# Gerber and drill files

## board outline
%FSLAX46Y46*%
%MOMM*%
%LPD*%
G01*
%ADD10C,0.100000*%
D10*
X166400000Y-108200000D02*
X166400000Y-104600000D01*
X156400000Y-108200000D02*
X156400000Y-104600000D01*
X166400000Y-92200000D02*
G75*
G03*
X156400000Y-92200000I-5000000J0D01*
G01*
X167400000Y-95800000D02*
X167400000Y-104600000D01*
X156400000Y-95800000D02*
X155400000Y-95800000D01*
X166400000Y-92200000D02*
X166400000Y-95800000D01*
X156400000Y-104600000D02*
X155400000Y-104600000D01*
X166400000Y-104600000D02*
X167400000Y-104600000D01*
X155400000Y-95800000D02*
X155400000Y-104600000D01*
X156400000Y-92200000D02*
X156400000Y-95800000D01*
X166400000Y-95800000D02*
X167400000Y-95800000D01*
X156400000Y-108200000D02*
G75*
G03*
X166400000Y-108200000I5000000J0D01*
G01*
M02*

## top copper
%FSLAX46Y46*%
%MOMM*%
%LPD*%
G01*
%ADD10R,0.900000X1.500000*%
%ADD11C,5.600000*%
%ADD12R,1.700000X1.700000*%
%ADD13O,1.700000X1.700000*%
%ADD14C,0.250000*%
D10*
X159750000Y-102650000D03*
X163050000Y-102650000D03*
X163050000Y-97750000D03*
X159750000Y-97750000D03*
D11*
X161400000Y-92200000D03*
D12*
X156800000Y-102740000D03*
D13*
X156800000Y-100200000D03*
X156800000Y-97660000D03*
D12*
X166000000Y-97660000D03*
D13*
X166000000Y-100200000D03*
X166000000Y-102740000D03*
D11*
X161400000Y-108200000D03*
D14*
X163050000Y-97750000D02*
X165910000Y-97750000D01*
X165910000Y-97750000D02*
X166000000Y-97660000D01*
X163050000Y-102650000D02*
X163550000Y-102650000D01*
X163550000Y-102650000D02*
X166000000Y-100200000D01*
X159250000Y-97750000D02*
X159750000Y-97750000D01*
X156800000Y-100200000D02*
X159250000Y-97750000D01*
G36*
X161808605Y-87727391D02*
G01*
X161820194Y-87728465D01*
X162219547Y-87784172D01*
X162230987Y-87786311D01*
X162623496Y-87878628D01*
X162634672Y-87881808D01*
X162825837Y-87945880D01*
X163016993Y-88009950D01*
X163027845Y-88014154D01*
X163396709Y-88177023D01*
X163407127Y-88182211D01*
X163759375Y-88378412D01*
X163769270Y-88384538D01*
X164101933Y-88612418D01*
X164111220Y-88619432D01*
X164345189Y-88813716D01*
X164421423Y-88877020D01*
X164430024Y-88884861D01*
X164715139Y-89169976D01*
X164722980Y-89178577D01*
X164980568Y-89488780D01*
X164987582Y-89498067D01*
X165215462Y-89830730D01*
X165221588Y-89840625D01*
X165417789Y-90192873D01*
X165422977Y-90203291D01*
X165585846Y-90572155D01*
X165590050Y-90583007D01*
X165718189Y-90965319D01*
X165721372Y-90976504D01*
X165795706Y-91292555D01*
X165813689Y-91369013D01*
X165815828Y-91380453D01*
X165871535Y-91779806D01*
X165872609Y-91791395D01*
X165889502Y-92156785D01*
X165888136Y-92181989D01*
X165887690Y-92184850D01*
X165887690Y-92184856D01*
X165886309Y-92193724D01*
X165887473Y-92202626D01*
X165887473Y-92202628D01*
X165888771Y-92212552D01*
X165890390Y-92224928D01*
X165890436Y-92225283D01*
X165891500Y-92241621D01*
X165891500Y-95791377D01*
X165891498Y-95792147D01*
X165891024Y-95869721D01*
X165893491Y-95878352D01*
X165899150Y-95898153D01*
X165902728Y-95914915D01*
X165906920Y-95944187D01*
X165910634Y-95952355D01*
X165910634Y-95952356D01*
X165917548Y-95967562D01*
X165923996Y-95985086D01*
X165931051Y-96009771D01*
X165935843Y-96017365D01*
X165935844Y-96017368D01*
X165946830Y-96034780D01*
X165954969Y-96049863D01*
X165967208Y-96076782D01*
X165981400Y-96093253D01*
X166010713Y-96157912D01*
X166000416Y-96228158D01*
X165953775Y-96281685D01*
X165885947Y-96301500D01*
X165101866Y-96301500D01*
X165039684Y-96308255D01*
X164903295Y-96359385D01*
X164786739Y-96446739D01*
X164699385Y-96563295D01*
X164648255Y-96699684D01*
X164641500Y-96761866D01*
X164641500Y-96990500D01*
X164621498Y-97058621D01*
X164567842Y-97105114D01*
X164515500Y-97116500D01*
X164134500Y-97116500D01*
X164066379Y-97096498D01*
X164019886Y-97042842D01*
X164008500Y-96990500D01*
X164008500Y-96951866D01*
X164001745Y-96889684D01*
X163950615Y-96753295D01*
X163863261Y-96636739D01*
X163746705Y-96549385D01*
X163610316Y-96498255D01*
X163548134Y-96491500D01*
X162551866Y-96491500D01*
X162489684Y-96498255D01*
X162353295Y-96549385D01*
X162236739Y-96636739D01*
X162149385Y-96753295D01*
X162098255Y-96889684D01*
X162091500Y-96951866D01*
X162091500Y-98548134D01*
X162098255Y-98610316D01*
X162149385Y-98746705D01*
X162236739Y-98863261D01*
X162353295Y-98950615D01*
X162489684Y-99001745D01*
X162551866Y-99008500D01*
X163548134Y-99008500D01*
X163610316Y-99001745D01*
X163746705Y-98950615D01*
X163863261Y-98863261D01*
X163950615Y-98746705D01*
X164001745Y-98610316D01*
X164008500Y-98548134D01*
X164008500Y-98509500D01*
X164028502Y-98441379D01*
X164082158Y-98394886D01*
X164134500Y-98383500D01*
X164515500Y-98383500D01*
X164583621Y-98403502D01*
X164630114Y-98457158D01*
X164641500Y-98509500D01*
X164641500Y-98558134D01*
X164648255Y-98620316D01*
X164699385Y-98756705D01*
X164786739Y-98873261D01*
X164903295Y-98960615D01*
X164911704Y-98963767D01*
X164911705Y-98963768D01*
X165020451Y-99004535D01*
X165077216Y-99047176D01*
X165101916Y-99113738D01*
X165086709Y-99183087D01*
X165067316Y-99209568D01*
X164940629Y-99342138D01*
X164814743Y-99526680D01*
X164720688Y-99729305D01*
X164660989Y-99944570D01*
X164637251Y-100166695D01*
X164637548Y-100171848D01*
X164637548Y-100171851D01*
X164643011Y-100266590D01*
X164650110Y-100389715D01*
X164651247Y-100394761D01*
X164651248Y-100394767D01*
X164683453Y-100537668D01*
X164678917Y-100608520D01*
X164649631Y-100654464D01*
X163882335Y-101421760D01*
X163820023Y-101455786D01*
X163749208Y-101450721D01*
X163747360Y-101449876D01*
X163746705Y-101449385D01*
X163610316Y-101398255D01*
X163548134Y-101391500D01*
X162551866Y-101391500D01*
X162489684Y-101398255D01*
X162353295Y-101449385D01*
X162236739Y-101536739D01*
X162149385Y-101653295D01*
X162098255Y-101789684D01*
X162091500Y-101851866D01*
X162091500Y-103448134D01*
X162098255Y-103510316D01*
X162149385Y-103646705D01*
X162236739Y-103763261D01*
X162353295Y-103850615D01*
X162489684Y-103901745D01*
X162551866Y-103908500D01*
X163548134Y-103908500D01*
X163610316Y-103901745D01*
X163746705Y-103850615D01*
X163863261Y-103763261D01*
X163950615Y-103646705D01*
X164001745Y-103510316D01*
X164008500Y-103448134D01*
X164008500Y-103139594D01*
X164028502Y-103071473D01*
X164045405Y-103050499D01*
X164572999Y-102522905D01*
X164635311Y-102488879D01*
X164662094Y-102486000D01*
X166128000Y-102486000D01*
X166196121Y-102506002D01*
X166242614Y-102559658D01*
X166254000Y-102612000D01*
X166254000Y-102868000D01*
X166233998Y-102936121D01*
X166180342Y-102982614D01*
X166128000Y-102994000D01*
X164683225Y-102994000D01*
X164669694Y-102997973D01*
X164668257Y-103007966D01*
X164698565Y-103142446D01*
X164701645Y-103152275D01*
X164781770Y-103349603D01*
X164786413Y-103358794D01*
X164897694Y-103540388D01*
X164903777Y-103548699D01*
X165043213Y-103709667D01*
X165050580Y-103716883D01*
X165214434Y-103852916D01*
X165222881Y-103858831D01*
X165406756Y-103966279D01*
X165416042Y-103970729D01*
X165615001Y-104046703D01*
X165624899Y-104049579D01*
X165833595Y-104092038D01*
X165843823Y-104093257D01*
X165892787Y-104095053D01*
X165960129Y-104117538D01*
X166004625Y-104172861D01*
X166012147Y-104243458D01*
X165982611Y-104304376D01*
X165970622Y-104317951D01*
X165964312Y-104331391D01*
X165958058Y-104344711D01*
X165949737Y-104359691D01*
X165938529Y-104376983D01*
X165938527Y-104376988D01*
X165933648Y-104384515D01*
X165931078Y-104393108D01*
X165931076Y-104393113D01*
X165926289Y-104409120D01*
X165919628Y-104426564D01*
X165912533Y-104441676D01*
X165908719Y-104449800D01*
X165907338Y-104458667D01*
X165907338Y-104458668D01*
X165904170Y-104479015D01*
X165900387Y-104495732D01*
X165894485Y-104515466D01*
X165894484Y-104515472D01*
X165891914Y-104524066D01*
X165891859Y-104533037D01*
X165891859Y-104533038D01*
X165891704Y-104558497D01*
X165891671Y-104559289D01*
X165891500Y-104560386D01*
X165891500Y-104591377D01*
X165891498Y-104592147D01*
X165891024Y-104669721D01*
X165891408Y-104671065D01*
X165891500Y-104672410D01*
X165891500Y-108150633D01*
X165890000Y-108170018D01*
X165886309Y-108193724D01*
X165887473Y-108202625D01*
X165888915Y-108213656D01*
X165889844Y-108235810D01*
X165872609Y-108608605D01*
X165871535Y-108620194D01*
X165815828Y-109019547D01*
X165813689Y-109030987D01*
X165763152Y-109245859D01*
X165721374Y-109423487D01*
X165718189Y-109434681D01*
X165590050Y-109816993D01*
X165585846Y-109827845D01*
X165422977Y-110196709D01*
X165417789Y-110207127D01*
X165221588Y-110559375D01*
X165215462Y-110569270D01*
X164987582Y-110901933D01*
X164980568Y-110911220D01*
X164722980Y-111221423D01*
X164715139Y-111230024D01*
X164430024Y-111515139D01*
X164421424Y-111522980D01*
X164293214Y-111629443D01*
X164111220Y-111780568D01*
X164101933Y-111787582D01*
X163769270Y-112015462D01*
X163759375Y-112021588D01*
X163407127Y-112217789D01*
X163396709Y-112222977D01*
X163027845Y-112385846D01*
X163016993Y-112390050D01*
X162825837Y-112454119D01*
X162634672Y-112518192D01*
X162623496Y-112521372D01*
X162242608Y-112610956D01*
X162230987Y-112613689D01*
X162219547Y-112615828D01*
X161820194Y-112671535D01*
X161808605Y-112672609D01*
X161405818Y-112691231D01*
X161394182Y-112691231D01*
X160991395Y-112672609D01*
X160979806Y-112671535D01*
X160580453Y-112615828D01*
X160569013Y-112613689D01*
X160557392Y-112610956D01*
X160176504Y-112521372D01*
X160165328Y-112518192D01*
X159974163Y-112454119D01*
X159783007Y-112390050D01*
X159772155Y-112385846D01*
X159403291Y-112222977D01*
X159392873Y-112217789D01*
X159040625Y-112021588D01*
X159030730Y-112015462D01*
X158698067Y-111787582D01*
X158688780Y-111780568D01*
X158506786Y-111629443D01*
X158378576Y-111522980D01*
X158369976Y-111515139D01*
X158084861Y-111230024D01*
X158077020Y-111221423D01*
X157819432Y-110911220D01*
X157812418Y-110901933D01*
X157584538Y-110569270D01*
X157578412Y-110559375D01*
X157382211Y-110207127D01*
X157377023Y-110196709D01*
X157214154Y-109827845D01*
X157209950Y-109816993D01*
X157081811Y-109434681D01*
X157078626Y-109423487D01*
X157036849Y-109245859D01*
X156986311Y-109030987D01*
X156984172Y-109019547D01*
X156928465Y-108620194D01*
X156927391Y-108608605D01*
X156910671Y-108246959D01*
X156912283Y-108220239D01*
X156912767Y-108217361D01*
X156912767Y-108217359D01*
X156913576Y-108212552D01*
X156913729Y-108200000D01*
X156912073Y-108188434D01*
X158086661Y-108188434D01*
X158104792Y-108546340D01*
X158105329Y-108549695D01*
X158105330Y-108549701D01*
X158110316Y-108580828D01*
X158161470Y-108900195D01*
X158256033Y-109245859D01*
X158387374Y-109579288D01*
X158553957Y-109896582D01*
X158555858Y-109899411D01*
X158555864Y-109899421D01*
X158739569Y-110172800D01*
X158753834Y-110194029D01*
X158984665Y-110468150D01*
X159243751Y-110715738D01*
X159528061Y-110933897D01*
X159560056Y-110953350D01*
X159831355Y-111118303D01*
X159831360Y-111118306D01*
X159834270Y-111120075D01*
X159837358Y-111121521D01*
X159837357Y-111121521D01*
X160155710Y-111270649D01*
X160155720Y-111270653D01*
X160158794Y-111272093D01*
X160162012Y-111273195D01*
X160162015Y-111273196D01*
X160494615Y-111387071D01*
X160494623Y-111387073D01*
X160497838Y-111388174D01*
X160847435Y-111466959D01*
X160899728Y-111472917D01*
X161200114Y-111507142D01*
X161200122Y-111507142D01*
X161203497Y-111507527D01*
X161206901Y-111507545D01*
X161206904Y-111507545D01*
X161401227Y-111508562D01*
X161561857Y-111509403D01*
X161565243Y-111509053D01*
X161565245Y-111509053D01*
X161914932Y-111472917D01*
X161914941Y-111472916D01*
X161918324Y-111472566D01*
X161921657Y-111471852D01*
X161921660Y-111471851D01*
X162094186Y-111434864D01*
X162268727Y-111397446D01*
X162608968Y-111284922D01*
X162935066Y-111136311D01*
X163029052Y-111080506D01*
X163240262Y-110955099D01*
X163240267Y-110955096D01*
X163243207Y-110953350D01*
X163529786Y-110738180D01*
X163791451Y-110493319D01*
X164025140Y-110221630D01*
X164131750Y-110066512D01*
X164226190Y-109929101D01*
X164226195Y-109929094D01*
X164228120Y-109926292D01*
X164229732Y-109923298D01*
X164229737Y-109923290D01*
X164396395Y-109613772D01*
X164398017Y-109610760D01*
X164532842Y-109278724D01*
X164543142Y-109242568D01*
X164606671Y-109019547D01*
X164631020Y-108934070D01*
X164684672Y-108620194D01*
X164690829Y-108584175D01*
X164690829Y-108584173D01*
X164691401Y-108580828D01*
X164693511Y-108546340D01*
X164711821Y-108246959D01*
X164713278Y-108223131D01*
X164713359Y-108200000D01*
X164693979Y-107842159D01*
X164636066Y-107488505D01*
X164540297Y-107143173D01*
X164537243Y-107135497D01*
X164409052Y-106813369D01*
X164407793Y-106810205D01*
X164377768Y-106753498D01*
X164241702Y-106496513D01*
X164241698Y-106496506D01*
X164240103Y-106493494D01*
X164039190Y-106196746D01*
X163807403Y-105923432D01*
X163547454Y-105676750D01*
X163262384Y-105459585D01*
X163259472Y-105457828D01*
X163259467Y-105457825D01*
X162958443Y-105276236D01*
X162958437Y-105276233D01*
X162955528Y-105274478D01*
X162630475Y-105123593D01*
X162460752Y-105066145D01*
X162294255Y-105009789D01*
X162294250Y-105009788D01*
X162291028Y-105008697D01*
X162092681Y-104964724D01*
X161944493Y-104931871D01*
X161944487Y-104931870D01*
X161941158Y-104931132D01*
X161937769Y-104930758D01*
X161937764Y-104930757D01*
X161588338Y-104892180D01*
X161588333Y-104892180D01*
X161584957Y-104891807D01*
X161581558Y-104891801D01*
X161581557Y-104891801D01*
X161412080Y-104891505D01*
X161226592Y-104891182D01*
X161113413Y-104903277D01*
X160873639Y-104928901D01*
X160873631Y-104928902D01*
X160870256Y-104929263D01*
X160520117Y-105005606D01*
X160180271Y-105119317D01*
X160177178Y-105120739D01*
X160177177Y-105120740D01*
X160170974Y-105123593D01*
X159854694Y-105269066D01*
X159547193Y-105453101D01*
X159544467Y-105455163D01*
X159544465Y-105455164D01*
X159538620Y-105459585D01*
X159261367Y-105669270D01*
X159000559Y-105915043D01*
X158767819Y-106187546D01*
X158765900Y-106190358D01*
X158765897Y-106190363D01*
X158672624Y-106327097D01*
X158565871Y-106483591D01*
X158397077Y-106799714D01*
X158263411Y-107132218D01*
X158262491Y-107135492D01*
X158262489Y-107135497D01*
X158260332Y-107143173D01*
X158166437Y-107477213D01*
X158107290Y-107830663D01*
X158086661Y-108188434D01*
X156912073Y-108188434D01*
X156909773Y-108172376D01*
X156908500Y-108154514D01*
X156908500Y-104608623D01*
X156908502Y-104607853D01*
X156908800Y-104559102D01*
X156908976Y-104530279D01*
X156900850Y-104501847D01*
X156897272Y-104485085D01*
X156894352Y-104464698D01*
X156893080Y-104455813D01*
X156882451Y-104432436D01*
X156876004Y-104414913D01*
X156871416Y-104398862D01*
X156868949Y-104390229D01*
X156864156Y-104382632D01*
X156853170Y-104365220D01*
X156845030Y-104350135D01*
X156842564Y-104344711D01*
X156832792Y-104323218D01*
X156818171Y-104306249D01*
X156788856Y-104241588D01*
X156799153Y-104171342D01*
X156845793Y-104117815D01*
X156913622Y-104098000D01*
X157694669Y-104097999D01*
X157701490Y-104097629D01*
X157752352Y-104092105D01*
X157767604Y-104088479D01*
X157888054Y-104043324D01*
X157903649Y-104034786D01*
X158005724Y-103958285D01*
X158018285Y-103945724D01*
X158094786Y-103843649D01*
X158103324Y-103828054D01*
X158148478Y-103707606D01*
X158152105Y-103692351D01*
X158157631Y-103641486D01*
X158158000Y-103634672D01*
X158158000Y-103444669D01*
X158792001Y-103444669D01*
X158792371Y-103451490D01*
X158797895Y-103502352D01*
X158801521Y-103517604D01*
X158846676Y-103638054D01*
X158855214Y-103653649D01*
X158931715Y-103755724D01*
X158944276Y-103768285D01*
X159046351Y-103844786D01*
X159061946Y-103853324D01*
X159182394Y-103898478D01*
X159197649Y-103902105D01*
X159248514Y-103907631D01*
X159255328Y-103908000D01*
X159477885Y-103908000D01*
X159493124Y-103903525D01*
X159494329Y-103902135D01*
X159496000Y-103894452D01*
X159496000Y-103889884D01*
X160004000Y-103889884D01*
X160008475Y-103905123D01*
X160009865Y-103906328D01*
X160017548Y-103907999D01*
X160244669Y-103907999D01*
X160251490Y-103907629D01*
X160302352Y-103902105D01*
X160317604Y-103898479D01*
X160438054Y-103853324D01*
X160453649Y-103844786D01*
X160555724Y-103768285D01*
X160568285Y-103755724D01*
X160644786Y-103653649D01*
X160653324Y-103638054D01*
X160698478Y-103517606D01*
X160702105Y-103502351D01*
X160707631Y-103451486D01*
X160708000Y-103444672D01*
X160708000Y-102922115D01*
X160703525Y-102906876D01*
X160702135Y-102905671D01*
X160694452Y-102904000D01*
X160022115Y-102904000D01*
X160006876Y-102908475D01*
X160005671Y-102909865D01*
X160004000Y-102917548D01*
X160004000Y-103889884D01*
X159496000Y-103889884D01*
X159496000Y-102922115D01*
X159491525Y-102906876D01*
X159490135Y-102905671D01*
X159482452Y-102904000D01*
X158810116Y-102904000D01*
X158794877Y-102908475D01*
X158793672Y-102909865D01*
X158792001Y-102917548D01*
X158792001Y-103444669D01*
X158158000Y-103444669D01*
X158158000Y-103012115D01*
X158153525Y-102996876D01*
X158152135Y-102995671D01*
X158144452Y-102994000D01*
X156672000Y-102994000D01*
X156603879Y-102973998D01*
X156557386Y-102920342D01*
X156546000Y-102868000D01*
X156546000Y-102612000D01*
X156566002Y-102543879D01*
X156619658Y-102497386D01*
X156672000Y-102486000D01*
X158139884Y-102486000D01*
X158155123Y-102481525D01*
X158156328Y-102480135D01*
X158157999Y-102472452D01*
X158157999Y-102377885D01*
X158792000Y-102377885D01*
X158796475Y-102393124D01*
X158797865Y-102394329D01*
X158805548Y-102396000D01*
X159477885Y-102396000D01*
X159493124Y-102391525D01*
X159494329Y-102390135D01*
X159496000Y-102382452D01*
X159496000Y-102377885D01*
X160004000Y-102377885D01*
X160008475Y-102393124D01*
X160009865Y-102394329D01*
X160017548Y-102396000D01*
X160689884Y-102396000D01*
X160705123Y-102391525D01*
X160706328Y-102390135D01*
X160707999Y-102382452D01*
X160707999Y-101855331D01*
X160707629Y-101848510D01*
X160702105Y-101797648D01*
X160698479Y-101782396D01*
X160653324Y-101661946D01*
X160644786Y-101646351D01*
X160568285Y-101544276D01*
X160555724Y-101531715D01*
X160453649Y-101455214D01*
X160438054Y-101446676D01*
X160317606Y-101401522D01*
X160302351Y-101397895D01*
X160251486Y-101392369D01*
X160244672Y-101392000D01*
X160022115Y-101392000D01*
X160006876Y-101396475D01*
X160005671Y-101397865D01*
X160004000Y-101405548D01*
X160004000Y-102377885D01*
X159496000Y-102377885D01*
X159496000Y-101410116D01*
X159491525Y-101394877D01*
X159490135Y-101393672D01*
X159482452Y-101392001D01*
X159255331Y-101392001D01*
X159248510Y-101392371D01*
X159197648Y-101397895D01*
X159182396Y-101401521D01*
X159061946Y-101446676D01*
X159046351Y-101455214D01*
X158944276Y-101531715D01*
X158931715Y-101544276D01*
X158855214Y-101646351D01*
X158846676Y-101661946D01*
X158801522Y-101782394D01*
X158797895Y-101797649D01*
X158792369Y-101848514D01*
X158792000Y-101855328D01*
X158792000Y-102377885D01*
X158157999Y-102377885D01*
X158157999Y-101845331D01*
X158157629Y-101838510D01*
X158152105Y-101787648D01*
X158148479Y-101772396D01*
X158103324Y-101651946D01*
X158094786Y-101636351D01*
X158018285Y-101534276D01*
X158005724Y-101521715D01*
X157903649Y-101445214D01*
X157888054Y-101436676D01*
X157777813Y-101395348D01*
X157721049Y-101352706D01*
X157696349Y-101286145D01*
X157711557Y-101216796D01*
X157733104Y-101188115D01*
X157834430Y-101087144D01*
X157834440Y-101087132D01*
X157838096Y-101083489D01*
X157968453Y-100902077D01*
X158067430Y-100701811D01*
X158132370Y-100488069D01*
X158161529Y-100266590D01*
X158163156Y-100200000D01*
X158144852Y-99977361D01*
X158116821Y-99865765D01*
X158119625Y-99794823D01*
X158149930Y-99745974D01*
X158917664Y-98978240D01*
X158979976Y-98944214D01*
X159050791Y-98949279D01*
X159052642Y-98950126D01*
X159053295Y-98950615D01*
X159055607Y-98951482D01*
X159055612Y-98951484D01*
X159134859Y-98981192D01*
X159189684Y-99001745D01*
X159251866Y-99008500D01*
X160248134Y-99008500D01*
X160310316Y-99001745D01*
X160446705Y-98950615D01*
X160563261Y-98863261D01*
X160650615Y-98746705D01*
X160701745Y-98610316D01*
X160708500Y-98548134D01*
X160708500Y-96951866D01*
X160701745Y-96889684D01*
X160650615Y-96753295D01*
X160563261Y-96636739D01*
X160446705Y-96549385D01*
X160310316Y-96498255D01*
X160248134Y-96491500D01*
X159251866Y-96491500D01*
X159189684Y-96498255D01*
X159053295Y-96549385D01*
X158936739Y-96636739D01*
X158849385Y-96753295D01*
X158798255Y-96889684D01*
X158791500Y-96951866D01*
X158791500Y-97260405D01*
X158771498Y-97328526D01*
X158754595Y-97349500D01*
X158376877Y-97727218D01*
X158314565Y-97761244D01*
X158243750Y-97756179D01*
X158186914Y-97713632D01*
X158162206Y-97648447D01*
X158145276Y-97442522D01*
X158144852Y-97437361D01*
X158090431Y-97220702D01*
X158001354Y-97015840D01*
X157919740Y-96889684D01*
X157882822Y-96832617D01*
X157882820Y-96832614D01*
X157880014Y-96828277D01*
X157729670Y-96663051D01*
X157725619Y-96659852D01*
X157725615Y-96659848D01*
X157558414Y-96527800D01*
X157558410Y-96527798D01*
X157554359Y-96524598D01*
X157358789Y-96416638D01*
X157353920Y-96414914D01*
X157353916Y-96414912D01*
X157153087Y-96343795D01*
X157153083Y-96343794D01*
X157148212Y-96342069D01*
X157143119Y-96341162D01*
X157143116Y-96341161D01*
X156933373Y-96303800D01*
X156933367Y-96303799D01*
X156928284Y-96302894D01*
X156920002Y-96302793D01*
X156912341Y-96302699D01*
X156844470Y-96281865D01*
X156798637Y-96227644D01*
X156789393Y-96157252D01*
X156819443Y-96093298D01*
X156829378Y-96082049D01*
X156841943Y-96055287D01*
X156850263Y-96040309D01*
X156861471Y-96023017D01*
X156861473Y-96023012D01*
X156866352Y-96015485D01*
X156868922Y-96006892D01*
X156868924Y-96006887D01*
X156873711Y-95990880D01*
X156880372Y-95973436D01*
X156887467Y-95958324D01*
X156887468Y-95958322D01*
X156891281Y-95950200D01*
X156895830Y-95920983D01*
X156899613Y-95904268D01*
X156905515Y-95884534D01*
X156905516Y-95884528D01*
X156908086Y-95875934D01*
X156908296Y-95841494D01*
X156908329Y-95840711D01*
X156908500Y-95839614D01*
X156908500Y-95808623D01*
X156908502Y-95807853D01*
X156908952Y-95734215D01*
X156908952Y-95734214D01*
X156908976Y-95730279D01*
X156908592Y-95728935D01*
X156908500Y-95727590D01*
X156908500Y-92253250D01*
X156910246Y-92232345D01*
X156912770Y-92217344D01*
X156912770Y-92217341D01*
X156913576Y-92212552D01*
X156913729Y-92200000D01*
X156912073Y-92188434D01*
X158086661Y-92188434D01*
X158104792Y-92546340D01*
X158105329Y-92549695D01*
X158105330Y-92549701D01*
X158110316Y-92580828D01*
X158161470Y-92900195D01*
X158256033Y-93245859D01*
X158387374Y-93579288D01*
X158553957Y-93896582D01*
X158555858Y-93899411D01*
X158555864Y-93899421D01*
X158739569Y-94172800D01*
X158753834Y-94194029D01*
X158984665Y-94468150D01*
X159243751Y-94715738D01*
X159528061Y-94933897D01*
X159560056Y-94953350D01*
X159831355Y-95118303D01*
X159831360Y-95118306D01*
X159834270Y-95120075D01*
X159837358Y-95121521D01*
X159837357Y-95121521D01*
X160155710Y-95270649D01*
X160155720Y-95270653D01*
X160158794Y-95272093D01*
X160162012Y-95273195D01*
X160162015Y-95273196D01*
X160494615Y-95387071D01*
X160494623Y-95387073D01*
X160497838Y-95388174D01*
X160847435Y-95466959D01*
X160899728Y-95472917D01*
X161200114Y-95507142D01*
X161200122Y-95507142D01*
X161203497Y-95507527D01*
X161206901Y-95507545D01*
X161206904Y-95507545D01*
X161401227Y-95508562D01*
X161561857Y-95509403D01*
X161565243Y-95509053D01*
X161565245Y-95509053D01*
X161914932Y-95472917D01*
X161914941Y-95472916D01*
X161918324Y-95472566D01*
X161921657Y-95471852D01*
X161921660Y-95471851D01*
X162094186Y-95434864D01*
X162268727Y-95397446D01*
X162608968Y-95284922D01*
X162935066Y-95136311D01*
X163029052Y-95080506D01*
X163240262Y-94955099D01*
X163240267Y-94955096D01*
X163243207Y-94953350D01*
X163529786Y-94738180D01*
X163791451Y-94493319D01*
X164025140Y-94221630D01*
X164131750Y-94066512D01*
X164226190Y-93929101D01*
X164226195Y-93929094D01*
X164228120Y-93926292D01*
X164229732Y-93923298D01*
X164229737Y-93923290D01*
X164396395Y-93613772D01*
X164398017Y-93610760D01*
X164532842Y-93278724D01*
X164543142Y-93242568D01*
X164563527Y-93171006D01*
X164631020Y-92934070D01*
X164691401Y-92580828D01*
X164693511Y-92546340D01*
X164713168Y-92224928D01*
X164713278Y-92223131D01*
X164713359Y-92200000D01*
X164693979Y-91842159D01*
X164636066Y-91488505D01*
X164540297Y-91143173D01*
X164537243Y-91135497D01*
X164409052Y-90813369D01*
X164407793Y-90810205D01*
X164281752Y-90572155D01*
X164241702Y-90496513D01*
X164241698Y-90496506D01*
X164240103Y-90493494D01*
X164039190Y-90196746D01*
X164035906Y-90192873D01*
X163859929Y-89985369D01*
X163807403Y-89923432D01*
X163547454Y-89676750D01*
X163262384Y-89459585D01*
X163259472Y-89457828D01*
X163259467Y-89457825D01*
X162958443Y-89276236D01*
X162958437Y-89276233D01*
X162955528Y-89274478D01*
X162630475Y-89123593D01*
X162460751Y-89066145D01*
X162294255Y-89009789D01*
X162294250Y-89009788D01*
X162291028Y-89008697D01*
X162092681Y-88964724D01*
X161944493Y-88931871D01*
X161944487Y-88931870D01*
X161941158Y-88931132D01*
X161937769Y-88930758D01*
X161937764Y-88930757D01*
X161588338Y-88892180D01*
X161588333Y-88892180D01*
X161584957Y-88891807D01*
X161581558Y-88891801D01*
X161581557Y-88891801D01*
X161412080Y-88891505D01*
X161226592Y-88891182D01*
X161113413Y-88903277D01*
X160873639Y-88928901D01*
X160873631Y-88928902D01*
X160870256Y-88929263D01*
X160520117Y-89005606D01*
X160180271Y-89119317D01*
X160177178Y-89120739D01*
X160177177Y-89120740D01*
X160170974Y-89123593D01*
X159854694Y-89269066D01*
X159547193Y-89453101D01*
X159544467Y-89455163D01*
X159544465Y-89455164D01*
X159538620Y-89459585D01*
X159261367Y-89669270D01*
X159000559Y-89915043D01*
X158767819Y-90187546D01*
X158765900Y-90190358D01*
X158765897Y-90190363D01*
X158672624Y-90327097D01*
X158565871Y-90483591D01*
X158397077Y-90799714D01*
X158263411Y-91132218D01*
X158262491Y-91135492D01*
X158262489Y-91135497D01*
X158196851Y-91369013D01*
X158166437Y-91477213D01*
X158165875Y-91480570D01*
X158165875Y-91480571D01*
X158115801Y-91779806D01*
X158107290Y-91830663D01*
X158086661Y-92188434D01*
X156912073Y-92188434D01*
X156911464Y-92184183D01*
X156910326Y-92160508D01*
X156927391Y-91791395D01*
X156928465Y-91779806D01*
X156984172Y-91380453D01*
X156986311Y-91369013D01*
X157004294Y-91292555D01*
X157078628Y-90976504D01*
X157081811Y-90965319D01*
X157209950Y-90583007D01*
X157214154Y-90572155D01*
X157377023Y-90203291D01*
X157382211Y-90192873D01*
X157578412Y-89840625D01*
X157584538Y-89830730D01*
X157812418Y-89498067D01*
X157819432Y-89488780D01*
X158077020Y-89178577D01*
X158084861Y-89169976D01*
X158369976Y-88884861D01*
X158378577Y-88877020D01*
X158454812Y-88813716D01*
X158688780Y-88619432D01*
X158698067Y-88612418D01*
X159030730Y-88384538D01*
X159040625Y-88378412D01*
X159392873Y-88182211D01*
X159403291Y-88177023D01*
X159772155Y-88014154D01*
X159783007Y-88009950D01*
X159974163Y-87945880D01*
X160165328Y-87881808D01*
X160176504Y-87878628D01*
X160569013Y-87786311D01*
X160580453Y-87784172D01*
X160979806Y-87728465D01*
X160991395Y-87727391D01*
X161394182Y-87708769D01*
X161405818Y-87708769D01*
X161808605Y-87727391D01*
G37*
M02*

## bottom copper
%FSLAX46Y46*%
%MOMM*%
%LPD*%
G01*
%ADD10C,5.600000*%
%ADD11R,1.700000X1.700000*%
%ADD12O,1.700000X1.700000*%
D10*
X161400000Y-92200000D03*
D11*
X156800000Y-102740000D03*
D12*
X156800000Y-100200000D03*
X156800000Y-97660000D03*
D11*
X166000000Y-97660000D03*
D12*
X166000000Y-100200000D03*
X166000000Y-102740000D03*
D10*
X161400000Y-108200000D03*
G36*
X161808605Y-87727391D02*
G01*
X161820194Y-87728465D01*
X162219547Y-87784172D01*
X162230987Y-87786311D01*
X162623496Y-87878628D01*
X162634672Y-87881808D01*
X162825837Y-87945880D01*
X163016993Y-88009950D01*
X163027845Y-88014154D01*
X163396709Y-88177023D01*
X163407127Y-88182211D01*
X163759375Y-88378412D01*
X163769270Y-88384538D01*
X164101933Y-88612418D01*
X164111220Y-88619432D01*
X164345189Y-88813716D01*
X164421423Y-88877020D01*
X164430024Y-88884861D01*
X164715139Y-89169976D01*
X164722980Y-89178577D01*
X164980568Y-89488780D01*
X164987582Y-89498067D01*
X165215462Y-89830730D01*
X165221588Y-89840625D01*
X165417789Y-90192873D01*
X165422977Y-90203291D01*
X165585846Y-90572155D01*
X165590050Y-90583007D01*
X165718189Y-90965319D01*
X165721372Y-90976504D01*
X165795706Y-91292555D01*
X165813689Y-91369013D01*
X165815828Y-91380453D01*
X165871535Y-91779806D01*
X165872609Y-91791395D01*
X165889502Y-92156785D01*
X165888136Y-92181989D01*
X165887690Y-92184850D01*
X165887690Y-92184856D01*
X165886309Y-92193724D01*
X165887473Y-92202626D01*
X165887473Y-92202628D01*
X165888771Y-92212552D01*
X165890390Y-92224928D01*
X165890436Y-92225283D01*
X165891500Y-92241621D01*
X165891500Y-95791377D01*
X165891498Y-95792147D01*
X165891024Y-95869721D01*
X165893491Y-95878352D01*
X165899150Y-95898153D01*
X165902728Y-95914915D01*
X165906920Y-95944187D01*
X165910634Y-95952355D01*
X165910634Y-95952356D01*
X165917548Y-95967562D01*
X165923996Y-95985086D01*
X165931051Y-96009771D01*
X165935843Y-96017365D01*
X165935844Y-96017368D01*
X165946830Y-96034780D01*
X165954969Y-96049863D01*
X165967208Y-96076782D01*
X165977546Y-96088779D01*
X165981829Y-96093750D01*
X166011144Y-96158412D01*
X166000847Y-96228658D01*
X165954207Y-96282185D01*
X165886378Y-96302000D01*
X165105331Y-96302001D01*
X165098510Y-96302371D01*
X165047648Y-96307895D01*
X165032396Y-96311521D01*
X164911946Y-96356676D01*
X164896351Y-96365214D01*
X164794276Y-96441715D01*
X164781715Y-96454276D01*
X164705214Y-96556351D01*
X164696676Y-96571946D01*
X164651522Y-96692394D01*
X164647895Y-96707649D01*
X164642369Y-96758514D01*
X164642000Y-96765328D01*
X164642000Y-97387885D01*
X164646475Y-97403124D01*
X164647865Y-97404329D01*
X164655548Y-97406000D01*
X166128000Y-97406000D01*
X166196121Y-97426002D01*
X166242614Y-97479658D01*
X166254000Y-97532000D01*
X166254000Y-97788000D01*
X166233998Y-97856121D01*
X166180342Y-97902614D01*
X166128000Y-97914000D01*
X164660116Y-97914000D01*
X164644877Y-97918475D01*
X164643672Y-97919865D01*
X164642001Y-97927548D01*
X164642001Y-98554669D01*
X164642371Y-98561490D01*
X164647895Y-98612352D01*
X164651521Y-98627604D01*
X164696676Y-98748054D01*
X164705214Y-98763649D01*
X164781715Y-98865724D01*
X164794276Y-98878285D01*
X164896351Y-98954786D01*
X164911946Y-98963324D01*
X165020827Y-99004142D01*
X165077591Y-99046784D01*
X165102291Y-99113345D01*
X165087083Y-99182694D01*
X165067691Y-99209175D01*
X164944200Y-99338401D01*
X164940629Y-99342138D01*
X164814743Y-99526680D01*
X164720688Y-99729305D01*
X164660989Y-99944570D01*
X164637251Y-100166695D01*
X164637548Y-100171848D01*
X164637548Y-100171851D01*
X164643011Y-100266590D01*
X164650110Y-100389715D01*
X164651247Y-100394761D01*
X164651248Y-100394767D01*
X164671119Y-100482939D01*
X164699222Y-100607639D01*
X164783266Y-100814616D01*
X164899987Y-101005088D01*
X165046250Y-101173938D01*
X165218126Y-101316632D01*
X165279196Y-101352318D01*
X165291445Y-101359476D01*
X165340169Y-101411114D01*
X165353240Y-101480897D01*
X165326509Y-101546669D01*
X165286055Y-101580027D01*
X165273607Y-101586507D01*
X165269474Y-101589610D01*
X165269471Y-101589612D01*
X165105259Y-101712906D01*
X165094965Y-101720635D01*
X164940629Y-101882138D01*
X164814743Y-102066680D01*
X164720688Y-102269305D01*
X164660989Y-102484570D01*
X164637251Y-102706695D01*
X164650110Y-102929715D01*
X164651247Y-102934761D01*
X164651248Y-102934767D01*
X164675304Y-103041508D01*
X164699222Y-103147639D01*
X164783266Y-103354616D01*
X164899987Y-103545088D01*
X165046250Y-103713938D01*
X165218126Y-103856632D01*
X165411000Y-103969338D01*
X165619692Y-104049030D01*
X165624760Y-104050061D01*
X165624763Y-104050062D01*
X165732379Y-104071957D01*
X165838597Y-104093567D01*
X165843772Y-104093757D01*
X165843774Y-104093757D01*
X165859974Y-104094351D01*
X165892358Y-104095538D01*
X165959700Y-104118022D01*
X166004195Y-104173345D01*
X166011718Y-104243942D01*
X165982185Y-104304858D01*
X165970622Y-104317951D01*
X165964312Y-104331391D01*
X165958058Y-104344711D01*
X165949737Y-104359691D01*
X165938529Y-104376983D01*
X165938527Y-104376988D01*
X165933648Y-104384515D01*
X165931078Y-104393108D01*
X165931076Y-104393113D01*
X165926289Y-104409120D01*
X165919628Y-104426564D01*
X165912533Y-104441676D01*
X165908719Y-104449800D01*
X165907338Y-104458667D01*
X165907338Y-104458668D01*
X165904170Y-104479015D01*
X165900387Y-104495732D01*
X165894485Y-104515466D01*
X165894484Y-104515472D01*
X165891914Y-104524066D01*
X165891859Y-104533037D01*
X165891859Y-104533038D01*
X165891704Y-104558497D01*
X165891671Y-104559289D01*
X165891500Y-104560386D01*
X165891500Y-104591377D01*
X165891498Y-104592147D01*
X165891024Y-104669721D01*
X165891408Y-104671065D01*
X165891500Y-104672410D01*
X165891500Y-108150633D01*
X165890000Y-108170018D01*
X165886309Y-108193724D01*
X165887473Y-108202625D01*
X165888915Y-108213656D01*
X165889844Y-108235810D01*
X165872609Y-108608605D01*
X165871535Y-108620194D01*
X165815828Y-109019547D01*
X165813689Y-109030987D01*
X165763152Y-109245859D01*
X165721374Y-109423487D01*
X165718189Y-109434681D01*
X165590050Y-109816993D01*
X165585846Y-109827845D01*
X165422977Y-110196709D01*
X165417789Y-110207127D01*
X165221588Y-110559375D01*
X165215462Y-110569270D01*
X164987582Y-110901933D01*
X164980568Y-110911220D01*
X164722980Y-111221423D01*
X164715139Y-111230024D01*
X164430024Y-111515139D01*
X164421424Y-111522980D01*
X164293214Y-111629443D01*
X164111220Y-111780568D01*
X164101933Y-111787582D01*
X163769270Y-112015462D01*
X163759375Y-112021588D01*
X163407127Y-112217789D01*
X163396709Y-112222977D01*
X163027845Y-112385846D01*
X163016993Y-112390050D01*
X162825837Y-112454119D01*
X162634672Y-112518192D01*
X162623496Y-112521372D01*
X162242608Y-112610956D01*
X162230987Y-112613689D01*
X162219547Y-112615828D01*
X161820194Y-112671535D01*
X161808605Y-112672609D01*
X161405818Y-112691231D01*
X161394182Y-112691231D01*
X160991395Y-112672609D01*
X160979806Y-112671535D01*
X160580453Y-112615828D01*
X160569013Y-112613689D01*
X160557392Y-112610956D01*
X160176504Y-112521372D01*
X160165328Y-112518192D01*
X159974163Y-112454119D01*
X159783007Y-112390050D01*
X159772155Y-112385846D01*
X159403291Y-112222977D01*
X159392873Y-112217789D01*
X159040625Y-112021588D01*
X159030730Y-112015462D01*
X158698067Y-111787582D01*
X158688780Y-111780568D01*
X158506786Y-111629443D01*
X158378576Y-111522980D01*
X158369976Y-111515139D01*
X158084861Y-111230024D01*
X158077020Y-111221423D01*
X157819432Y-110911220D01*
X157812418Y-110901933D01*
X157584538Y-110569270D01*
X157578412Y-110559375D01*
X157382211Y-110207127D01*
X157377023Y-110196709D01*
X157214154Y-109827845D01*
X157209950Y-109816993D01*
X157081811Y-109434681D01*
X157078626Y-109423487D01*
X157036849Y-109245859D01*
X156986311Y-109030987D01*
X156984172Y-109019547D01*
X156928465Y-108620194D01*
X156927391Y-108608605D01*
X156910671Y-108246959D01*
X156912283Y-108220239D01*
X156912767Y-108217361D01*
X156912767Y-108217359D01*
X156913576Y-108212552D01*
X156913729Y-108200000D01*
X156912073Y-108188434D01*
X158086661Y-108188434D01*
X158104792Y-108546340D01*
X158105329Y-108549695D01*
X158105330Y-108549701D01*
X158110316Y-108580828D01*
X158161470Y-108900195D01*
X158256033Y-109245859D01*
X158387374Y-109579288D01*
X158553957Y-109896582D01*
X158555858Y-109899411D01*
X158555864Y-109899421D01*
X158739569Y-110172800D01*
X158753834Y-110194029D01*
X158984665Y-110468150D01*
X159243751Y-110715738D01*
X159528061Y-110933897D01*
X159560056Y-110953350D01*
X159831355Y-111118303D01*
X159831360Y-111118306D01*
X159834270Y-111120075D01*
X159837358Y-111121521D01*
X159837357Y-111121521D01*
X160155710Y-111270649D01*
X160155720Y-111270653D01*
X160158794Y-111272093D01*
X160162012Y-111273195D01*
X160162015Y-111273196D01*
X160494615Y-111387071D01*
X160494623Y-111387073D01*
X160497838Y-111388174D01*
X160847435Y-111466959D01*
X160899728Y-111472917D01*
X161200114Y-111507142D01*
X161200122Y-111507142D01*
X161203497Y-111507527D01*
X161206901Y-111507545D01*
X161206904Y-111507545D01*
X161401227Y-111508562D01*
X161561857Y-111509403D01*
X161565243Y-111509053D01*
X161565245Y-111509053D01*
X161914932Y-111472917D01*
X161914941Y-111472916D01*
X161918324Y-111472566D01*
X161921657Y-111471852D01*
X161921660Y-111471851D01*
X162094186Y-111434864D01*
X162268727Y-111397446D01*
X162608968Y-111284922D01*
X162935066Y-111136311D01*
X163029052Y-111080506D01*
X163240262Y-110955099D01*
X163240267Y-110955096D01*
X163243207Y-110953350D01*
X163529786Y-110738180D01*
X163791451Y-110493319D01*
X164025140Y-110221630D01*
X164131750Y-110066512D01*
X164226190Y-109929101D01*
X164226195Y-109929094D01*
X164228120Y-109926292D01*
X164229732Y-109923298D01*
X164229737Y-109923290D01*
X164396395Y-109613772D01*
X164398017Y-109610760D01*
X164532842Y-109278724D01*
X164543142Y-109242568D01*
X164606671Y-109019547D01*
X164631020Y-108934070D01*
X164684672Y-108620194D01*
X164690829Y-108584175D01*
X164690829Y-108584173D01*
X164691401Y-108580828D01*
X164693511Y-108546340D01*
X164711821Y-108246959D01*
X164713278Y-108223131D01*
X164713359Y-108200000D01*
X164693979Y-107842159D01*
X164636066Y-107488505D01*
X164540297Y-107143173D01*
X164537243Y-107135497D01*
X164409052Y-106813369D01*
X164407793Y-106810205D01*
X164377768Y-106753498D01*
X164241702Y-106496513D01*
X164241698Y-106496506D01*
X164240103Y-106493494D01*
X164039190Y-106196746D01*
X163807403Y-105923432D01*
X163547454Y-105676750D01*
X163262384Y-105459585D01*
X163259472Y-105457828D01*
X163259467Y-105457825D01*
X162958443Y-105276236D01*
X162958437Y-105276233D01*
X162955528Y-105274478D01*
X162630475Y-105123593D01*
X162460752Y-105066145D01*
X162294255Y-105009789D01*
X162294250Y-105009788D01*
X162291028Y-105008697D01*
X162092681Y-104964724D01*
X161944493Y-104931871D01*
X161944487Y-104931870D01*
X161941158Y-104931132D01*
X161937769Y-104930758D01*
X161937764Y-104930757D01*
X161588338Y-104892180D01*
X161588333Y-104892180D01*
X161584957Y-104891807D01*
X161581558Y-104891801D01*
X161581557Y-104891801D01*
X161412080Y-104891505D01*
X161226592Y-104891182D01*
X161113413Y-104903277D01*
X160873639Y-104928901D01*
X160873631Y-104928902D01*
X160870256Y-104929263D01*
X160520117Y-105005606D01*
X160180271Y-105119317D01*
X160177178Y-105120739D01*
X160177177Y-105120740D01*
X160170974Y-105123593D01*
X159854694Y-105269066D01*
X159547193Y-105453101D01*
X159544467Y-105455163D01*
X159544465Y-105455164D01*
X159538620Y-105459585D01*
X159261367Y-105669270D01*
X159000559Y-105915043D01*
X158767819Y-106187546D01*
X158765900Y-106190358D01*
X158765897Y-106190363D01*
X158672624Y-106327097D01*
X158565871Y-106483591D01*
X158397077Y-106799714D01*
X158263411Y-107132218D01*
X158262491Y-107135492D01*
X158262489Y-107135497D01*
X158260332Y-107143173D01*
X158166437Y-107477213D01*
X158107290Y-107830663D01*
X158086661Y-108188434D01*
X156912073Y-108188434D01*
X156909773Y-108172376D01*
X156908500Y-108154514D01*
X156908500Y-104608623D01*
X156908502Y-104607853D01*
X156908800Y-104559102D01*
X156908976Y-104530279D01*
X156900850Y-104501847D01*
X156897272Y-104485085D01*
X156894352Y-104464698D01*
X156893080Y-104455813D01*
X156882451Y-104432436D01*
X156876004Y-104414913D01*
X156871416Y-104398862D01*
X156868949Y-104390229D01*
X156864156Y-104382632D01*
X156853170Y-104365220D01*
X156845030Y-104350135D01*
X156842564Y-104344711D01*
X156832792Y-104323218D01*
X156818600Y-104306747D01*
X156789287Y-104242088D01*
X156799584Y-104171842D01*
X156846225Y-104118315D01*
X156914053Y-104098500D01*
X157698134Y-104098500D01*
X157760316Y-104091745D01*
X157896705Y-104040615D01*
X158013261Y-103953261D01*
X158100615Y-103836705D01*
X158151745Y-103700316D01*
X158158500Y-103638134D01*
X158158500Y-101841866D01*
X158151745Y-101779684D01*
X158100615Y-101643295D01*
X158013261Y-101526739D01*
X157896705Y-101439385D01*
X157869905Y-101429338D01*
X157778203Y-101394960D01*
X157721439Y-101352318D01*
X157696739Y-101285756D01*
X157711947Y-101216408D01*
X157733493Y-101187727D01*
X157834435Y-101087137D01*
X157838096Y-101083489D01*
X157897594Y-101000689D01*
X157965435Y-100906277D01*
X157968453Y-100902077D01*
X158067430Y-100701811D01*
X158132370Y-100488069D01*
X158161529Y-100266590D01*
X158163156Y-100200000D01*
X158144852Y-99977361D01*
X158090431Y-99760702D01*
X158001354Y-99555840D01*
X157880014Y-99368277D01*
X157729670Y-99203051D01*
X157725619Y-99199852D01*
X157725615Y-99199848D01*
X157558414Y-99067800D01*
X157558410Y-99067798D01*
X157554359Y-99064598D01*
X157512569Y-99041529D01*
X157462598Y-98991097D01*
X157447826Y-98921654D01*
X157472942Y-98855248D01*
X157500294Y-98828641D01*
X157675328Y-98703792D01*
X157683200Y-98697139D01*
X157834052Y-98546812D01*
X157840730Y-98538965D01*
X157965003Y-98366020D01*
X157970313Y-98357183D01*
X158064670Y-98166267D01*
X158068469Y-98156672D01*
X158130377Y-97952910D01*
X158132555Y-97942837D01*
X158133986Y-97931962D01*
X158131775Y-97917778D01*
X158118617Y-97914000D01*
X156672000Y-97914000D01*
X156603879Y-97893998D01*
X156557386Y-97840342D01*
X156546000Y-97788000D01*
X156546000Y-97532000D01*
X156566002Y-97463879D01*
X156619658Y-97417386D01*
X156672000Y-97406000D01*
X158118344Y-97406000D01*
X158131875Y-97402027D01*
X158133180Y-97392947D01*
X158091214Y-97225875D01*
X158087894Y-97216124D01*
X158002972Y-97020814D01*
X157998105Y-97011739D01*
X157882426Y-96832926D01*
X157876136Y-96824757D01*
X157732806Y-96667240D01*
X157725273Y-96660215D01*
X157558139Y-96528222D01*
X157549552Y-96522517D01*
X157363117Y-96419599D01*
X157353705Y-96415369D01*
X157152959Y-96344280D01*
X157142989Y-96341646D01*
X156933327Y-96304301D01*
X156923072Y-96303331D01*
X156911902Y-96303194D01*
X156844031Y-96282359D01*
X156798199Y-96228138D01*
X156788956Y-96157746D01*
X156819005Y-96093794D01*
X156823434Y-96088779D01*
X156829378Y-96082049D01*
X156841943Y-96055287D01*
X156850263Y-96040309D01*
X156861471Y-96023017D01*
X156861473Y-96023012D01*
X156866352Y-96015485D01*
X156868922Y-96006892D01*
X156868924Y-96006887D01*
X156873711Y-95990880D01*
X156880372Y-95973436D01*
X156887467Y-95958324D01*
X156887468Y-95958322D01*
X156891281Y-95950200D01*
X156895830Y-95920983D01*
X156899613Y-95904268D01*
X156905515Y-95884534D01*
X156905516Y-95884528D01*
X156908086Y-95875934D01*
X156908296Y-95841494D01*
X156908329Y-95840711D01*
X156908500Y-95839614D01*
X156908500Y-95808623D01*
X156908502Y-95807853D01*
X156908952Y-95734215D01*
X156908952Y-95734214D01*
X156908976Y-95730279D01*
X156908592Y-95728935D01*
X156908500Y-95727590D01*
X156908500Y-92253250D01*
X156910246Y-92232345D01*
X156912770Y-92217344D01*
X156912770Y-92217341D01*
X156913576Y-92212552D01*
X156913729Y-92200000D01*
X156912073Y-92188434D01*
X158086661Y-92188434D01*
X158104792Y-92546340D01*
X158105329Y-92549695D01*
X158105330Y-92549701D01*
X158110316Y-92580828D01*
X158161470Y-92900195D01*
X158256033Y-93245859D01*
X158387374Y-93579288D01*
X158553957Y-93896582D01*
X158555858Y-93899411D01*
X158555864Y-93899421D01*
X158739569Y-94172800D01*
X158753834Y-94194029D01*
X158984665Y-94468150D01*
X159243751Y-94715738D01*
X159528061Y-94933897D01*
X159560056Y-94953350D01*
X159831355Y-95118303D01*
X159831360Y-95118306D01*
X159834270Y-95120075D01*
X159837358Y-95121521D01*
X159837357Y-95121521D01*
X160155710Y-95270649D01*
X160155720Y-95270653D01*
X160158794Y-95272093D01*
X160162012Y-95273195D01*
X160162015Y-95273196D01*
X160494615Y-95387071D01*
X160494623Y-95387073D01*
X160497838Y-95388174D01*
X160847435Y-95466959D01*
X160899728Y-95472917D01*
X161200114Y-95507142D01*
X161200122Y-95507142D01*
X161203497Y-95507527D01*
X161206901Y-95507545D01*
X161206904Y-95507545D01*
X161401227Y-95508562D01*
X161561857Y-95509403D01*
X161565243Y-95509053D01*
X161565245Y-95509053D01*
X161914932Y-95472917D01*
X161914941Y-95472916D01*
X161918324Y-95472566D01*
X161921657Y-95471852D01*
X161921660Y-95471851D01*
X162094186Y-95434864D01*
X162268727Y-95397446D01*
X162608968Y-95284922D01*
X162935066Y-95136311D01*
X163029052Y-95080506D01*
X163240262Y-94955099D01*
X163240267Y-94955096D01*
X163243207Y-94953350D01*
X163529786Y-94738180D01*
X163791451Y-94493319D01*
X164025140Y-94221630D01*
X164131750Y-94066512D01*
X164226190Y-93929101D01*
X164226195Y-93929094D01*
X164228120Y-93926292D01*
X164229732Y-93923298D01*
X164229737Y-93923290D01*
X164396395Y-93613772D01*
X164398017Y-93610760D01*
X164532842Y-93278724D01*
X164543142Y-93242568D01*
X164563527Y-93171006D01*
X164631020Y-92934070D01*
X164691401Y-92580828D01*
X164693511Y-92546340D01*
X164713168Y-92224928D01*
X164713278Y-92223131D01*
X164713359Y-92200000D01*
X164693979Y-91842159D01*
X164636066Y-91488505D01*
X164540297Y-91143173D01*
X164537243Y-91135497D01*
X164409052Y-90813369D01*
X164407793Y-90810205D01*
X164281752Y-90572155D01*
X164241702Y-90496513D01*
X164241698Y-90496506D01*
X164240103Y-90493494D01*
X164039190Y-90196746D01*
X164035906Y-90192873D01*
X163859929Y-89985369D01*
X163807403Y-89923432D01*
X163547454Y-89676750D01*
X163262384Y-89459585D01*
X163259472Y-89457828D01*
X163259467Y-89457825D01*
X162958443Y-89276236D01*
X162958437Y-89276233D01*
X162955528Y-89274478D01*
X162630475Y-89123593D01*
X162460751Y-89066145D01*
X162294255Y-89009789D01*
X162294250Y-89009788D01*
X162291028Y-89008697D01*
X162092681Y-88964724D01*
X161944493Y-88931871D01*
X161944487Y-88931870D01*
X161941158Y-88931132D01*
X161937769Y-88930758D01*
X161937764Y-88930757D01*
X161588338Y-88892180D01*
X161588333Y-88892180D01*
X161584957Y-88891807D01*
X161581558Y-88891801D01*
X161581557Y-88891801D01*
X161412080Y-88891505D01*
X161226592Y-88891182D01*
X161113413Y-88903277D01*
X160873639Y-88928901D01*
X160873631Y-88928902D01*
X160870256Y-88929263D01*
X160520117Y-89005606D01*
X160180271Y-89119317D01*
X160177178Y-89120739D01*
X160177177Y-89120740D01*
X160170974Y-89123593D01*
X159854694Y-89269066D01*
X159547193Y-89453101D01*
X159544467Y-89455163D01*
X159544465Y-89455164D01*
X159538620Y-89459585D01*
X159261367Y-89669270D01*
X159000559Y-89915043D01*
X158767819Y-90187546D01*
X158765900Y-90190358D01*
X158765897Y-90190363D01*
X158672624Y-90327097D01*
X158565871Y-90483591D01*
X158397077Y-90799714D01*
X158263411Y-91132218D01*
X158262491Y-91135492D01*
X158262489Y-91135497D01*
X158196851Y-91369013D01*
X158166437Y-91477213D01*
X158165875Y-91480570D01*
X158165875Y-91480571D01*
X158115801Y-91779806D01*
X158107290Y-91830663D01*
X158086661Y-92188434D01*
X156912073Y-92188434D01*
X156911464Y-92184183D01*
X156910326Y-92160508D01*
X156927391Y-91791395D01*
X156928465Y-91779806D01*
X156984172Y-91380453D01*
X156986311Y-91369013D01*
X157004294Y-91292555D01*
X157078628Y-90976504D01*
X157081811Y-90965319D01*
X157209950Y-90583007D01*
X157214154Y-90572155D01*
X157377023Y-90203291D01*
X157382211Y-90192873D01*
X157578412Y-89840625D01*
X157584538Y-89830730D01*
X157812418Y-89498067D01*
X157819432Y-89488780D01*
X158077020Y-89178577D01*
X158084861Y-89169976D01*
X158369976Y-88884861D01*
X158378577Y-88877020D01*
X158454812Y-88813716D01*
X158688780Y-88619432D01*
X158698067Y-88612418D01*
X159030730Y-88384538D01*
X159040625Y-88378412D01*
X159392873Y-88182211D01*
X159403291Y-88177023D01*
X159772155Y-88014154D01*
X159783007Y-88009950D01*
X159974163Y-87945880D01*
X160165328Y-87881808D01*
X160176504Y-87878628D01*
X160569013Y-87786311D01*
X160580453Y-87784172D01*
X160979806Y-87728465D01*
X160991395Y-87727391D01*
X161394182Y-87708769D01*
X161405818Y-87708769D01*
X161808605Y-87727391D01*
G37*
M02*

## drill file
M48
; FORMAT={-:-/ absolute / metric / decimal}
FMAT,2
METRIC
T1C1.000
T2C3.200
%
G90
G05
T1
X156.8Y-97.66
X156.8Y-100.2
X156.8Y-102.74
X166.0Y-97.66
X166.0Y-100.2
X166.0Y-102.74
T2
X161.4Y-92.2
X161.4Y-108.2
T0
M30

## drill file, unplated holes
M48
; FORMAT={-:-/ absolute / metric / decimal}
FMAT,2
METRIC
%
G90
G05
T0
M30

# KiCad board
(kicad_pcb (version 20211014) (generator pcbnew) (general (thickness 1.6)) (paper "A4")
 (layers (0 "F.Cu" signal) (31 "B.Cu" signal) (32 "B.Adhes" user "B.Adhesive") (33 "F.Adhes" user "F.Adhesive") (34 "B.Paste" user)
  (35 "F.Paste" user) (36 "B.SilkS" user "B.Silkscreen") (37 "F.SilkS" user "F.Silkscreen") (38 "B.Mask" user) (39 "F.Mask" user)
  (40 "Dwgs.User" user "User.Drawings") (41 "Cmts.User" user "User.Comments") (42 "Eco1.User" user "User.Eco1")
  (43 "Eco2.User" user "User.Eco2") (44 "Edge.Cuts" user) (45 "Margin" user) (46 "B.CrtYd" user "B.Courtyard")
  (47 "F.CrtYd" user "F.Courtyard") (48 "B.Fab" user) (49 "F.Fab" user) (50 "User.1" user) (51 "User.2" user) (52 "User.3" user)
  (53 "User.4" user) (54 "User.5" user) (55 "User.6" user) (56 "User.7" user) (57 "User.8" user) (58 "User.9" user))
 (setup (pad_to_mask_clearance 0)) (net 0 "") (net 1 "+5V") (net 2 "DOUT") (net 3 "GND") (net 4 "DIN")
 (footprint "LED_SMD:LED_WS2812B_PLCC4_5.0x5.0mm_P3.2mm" (layer "F.Cu") (at 161.4 100.2 90)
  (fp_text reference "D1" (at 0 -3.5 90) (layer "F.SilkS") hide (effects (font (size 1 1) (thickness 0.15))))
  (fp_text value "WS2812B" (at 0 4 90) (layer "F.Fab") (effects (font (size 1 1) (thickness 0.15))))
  (pad "1" smd rect (at -2.45 -1.65 90) (size 1.5 0.9) (layers "F.Cu" "F.Paste" "F.Mask") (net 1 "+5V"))
  (pad "2" smd rect (at -2.45 1.65 90) (size 1.5 0.9) (layers "F.Cu" "F.Paste" "F.Mask") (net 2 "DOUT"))
  (pad "3" smd rect (at 2.45 1.65 90) (size 1.5 0.9) (layers "F.Cu" "F.Paste" "F.Mask") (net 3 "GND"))
  (pad "4" smd rect (at 2.45 -1.65 90) (size 1.5 0.9) (layers "F.Cu" "F.Paste" "F.Mask") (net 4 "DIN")))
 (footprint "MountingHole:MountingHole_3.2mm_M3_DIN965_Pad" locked (layer "F.Cu") (at 161.4 92.2)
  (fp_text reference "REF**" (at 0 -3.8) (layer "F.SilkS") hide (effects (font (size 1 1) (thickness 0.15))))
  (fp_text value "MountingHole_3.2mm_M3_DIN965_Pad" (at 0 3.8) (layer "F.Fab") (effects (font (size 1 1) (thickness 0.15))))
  (pad "1" thru_hole circle locked (at 0 0) (size 5.6 5.6) (drill 3.2) (layers *.Cu *.Mask)))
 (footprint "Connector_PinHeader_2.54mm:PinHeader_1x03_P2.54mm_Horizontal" (layer "F.Cu") (at 156.8 102.74 180)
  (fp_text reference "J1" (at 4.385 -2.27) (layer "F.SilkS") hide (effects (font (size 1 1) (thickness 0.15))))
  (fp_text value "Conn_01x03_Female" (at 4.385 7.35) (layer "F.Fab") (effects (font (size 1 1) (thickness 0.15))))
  (pad "1" thru_hole rect (at 0 0 180) (size 1.7 1.7) (drill 1) (layers *.Cu *.Mask) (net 1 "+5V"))
  (pad "2" thru_hole oval (at 0 2.54 180) (size 1.7 1.7) (drill 1) (layers *.Cu *.Mask) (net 4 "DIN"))
  (pad "3" thru_hole oval (at 0 5.08 180) (size 1.7 1.7) (drill 1) (layers *.Cu *.Mask) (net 3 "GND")))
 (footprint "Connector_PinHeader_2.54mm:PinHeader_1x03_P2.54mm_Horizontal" (layer "F.Cu") (at 166 97.66)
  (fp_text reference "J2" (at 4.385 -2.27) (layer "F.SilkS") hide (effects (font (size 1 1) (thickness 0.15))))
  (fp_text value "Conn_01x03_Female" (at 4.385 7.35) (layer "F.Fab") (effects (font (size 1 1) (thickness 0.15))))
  (pad "1" thru_hole rect (at 0 0) (size 1.7 1.7) (drill 1) (layers *.Cu *.Mask) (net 3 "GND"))
  (pad "2" thru_hole oval (at 0 2.54) (size 1.7 1.7) (drill 1) (layers *.Cu *.Mask) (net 2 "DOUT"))
  (pad "3" thru_hole oval (at 0 5.08) (size 1.7 1.7) (drill 1) (layers *.Cu *.Mask) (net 1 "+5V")))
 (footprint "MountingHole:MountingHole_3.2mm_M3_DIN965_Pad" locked (layer "F.Cu") (at 161.4 108.2)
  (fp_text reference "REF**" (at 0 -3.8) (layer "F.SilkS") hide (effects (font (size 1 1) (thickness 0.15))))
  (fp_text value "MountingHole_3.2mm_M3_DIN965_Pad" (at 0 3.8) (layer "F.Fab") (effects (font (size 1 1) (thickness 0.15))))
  (pad "1" thru_hole circle locked (at 0 0) (size 5.6 5.6) (drill 3.2) (layers *.Cu *.Mask)))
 (gr_line (start 166.4 108.2) (end 166.4 104.6) (layer "Edge.Cuts") (width 0.1))
 (gr_line (start 156.4 108.2) (end 156.4 104.6) (layer "Edge.Cuts") (width 0.1))
 (gr_arc (start 156.4 92.2) (mid 161.4 87.2) (end 166.4 92.2) (layer "Edge.Cuts") (width 0.1))
 (gr_line (start 167.4 95.8) (end 167.4 104.6) (layer "Edge.Cuts") (width 0.1))
 (gr_line (start 156.4 95.8) (end 155.4 95.8) (layer "Edge.Cuts") (width 0.1))
 (gr_line (start 166.4 92.2) (end 166.4 95.8) (layer "Edge.Cuts") (width 0.1))
 (gr_line (start 156.4 104.6) (end 155.4 104.6) (layer "Edge.Cuts") (width 0.1))
 (gr_line (start 166.4 104.6) (end 167.4 104.6) (layer "Edge.Cuts") (width 0.1))
 (gr_line (start 155.4 95.8) (end 155.4 104.6) (layer "Edge.Cuts") (width 0.1))
 (gr_line (start 156.4 92.2) (end 156.4 95.8) (layer "Edge.Cuts") (width 0.1))
 (gr_line (start 166.4 95.8) (end 167.4 95.8) (layer "Edge.Cuts") (width 0.1))
 (gr_arc (start 166.4 108.2) (mid 161.4 113.2) (end 156.4 108.2) (layer "Edge.Cuts") (width 0.1))
 (segment (start 163.05 97.75) (end 165.91 97.75) (width 0.25) (layer "F.Cu") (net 3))
 (segment (start 165.91 97.75) (end 166 97.66) (width 0.25) (layer "F.Cu") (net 3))
 (segment (start 163.05 102.65) (end 163.55 102.65) (width 0.25) (layer "F.Cu") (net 2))
 (segment (start 163.55 102.65) (end 166 100.2) (width 0.25) (layer "F.Cu") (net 2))
 (segment (start 159.25 97.75) (end 159.75 97.75) (width 0.25) (layer "F.Cu") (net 4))
 (segment (start 156.8 100.2) (end 159.25 97.75) (width 0.25) (layer "F.Cu") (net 4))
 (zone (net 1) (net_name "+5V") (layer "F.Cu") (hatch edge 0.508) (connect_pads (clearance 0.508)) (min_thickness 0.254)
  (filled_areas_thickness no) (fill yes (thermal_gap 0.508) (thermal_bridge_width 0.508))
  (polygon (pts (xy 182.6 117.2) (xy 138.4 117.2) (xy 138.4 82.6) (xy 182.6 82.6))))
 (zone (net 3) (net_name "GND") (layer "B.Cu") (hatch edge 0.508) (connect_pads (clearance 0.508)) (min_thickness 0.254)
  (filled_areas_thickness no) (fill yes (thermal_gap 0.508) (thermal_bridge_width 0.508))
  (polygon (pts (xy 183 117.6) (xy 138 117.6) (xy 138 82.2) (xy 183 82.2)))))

